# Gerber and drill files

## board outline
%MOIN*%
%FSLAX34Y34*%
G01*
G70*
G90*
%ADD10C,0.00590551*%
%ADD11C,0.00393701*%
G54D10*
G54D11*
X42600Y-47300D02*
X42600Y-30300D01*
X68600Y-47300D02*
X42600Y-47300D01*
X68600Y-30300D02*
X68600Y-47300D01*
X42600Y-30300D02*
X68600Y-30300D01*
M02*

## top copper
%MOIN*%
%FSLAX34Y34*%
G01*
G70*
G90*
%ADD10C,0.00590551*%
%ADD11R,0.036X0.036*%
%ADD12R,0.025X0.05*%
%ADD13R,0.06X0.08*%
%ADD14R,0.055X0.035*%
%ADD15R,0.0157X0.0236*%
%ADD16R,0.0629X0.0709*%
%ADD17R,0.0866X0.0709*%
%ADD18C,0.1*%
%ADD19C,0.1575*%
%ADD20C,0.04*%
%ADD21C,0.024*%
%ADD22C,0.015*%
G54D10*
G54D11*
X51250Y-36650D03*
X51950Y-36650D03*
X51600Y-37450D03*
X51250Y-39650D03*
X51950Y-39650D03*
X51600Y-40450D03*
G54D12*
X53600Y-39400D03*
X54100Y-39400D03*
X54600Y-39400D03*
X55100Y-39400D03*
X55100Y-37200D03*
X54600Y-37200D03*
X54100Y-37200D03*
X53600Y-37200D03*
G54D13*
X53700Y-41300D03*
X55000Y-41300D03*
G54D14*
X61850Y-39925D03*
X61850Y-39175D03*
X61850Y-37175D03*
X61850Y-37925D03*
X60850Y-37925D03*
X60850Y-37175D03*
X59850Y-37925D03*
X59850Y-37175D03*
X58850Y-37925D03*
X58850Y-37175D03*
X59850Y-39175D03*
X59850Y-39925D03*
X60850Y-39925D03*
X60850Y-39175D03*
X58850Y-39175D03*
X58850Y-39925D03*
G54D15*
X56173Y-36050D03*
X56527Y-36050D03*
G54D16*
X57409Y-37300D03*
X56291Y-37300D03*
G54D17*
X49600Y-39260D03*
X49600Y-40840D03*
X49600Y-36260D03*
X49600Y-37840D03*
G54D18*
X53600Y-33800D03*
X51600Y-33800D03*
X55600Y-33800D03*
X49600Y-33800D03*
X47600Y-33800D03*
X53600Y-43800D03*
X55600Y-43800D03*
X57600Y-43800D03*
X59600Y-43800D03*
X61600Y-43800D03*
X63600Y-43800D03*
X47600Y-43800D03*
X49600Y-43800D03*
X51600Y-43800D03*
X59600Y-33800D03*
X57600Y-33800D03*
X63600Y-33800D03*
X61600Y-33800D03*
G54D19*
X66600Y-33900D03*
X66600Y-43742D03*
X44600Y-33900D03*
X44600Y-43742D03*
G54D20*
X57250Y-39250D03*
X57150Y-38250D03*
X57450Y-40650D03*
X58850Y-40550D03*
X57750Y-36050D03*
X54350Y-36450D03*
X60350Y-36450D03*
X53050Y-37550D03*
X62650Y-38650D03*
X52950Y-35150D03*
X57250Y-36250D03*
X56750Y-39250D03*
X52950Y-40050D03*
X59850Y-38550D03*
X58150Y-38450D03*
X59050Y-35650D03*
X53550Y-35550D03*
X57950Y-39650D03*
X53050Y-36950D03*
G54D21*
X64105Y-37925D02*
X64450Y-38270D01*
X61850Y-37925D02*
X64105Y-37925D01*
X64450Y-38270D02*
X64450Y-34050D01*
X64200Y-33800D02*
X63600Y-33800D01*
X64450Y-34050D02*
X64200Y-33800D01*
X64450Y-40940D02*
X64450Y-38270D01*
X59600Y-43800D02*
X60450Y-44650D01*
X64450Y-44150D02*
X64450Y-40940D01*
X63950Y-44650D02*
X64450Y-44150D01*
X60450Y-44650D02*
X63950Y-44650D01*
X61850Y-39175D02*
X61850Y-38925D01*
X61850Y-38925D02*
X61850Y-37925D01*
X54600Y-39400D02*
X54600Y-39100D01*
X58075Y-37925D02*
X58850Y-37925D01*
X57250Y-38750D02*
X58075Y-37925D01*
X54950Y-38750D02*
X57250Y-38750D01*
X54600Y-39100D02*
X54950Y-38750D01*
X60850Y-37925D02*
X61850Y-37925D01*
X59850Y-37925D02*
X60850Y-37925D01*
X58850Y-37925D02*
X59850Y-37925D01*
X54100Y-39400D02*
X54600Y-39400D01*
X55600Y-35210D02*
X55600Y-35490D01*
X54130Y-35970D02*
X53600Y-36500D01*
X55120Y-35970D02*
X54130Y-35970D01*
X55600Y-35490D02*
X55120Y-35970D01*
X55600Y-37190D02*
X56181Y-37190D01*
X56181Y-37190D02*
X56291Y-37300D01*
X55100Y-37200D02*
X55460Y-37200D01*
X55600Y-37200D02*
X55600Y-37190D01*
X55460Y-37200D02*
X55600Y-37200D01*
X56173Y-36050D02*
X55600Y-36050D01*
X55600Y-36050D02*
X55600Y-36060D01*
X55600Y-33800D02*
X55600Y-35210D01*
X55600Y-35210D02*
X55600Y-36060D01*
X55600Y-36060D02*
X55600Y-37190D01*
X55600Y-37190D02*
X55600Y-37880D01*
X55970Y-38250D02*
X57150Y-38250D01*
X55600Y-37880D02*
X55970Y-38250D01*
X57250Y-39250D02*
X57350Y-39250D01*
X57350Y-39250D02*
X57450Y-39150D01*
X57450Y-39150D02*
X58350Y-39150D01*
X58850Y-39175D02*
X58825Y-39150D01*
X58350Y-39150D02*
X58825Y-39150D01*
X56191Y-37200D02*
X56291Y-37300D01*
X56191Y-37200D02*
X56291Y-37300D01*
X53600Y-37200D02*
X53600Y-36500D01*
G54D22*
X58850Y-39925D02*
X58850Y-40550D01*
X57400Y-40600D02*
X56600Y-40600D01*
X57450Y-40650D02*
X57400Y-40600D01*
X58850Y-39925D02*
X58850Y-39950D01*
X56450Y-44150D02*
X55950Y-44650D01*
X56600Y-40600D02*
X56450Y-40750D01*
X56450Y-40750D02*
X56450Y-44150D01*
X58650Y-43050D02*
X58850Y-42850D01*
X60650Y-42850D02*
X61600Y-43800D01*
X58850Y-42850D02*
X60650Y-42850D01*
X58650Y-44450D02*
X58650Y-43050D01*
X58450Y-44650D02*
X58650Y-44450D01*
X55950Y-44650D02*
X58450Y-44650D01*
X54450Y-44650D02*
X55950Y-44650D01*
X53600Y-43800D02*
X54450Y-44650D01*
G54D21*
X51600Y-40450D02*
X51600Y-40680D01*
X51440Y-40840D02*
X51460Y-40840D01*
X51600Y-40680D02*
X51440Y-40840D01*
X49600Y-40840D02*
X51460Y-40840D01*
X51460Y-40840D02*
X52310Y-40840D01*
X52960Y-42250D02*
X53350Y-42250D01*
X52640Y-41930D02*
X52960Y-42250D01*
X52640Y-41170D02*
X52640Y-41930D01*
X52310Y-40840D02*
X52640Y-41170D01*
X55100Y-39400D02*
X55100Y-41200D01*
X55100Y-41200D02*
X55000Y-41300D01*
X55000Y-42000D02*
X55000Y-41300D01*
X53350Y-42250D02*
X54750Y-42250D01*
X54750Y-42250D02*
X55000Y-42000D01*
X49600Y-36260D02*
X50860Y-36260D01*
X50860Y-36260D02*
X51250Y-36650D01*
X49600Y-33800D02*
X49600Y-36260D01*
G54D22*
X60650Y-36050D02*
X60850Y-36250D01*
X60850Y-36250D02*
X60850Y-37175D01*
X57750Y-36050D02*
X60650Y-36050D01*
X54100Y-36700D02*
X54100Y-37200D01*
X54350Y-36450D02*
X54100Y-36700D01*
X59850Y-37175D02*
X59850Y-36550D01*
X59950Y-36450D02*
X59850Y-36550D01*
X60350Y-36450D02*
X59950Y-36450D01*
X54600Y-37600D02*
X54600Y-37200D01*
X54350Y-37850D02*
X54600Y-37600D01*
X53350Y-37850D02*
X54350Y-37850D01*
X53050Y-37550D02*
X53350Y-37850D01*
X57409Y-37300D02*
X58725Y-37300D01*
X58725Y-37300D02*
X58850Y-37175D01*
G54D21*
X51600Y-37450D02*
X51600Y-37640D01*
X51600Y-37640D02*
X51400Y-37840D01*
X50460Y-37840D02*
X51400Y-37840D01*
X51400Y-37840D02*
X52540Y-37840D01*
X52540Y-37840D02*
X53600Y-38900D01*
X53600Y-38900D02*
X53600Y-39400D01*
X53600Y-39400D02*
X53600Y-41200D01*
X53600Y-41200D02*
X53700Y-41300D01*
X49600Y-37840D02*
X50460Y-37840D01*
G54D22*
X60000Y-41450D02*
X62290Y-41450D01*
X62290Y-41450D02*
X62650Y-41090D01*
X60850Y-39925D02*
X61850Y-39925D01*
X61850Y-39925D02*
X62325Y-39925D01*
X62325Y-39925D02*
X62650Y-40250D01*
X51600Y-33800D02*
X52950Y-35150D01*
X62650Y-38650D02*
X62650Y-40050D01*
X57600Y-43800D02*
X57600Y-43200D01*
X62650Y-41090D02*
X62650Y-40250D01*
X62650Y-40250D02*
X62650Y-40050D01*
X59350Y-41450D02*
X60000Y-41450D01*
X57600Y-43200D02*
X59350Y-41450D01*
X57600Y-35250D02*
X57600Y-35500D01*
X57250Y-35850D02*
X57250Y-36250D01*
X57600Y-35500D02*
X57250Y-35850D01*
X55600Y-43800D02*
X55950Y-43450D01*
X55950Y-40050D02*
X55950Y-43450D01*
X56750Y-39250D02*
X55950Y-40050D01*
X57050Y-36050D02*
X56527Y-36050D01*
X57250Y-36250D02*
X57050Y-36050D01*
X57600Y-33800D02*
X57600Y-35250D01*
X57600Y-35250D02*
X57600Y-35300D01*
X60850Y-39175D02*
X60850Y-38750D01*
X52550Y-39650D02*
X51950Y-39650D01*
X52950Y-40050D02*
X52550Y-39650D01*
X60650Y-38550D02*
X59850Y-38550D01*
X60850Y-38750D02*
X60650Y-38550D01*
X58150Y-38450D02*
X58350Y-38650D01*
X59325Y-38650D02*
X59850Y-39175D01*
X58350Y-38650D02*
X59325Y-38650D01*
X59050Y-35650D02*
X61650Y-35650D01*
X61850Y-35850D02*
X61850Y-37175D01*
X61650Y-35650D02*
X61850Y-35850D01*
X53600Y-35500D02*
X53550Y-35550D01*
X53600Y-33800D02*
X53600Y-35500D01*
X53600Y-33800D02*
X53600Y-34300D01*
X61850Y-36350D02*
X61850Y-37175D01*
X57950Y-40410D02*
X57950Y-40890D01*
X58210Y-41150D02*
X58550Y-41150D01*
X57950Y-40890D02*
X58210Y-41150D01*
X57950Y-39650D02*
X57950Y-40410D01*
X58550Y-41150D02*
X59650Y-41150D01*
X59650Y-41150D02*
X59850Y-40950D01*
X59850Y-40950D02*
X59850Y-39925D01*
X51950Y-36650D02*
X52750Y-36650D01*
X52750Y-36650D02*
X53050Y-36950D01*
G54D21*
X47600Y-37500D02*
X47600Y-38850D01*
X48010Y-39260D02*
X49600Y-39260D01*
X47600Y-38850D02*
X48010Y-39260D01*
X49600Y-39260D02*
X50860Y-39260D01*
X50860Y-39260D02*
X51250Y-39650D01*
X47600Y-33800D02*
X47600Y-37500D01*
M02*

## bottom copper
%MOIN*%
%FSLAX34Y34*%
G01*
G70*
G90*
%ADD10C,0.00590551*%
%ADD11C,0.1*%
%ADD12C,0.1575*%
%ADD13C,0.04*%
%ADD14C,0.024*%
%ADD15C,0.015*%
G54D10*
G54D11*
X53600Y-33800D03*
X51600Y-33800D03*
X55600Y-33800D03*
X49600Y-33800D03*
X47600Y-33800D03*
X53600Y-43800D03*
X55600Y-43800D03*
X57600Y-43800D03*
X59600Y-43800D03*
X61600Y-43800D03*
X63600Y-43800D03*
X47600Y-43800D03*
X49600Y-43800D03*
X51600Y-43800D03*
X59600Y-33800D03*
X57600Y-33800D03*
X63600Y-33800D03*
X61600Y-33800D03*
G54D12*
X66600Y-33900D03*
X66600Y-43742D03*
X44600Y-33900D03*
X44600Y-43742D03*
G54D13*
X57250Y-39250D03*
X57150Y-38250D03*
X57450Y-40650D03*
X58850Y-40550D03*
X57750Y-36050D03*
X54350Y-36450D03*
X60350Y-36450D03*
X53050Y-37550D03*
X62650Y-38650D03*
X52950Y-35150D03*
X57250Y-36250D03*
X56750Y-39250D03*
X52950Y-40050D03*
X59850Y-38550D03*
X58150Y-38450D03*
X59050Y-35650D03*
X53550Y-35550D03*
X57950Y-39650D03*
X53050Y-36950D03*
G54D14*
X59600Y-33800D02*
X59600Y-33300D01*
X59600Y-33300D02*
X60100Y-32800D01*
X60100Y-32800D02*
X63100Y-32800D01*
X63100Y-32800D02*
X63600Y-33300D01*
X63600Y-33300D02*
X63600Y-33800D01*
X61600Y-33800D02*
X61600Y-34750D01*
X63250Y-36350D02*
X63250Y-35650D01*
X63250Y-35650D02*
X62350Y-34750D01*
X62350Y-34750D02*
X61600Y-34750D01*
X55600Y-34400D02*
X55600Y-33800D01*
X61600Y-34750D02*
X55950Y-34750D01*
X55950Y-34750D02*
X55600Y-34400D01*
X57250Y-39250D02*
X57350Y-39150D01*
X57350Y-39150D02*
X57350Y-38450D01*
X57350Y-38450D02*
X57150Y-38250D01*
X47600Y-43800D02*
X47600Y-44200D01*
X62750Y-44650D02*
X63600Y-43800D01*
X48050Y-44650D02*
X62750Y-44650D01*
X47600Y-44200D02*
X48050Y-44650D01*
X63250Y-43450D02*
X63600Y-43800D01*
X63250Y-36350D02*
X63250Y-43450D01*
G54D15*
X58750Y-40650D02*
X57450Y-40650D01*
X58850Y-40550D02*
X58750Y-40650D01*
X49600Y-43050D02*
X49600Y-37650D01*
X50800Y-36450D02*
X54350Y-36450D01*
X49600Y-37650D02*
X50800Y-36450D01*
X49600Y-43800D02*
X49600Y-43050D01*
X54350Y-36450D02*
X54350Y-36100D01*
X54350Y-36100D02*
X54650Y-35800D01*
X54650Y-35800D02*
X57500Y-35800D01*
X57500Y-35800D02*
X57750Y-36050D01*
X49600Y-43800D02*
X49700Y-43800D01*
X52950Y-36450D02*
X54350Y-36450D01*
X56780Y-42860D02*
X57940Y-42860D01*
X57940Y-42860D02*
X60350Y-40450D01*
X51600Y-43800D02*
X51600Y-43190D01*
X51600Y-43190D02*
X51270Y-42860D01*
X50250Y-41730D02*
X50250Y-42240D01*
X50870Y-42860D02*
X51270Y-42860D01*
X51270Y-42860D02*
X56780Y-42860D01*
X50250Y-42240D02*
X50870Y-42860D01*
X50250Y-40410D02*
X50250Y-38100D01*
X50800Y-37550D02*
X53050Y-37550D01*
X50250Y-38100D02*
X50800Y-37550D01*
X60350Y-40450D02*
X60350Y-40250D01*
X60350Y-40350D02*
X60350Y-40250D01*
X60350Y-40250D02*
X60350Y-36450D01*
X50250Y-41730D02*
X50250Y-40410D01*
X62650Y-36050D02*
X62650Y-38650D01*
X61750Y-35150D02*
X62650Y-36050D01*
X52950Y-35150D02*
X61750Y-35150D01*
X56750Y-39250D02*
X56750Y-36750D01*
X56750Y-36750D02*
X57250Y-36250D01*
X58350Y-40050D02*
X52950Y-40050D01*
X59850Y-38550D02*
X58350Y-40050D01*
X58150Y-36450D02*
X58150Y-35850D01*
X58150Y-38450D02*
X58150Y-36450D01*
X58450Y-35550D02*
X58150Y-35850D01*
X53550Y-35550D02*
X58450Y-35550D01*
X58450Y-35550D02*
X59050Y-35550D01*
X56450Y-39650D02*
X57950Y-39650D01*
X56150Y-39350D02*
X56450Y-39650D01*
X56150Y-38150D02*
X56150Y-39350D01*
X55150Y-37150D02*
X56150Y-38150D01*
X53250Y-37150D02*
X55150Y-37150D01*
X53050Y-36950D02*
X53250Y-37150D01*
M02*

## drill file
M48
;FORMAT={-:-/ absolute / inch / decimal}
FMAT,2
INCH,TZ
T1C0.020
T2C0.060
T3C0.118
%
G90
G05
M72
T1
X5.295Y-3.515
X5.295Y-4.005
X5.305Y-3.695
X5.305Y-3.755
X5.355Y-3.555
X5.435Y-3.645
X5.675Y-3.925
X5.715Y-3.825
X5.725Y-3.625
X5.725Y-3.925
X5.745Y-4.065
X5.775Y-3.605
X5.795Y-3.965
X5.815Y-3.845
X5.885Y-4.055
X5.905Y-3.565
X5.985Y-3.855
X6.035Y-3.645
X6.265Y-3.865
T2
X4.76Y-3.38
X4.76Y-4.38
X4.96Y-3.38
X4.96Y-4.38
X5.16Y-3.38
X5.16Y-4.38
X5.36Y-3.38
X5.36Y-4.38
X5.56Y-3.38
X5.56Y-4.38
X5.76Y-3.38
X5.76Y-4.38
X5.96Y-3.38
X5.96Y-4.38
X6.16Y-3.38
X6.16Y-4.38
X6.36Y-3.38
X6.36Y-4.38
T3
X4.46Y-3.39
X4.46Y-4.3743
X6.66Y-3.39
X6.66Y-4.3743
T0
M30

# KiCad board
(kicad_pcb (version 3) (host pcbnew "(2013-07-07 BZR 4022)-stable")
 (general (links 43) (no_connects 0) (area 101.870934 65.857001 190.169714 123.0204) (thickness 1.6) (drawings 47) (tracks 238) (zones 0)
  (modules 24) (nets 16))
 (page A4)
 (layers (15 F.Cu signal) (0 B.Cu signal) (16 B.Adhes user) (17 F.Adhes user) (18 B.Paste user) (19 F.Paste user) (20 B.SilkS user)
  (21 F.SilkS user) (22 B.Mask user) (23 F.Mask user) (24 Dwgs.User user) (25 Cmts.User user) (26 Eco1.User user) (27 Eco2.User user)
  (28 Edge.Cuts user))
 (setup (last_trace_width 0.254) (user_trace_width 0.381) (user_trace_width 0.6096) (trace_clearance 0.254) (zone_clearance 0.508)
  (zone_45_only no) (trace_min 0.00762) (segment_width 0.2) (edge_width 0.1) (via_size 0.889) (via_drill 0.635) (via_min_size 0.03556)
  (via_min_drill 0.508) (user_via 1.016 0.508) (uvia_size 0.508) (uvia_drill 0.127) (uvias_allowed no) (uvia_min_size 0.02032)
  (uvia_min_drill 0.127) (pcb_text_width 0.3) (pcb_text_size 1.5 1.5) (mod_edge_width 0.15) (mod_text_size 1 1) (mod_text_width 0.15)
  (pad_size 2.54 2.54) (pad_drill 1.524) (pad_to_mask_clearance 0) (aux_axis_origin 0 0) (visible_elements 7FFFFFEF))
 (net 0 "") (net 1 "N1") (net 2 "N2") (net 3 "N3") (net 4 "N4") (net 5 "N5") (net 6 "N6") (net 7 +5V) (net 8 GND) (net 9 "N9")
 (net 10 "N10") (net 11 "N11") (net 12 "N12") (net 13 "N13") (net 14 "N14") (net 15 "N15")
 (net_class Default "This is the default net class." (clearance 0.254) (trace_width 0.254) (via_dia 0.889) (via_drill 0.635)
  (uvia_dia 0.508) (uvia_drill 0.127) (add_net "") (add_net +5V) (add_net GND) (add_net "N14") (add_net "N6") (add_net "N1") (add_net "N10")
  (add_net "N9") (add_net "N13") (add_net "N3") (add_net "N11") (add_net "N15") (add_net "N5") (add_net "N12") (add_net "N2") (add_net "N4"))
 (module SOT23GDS (layer F.Cu) (at 131.064 94.107)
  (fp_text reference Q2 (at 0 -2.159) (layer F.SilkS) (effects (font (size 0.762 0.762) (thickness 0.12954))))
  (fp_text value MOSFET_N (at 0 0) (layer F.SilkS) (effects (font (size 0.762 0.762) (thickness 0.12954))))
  (pad S smd rect (at -0.889 -1.016) (size 0.9144 0.9144) (layers F.Cu F.Paste F.Mask) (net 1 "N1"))
  (pad G smd rect (at 0.889 -1.016) (size 0.9144 0.9144) (layers F.Cu F.Paste F.Mask) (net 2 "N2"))
  (pad D smd rect (at 0 1.016) (size 0.9144 0.9144) (layers F.Cu F.Paste F.Mask) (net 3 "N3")))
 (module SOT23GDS (layer F.Cu) (at 131.064 101.727)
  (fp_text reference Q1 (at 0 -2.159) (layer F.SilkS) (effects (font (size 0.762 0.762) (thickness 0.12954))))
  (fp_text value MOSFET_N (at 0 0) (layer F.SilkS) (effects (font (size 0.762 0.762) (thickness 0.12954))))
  (pad S smd rect (at -0.889 -1.016) (size 0.9144 0.9144) (layers F.Cu F.Paste F.Mask) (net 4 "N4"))
  (pad G smd rect (at 0.889 -1.016) (size 0.9144 0.9144) (layers F.Cu F.Paste F.Mask) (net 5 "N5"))
  (pad D smd rect (at 0 1.016) (size 0.9144 0.9144) (layers F.Cu F.Paste F.Mask) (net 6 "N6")))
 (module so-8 (layer F.Cu) (at 138.049 97.282)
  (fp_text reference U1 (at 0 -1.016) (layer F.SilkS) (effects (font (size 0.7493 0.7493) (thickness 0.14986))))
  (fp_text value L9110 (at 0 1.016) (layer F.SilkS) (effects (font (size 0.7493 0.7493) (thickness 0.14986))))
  (pad 1 smd rect (at -1.905 2.794) (size 0.635 1.27) (layers F.Cu F.Paste F.Mask) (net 3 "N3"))
  (pad 2 smd rect (at -0.635 2.794) (size 0.635 1.27) (layers F.Cu F.Paste F.Mask) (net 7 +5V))
  (pad 3 smd rect (at 0.635 2.794) (size 0.635 1.27) (layers F.Cu F.Paste F.Mask) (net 7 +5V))
  (pad 4 smd rect (at 1.905 2.794) (size 0.635 1.27) (layers F.Cu F.Paste F.Mask) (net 6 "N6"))
  (pad 5 smd rect (at 1.905 -2.794) (size 0.635 1.27) (layers F.Cu F.Paste F.Mask) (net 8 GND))
  (pad 6 smd rect (at 0.635 -2.794) (size 0.635 1.27) (layers F.Cu F.Paste F.Mask) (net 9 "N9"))
  (pad 7 smd rect (at -0.635 -2.794) (size 0.635 1.27) (layers F.Cu F.Paste F.Mask) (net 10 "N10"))
  (pad 8 smd rect (at -1.905 -2.794) (size 0.635 1.27) (layers F.Cu F.Paste F.Mask) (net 8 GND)))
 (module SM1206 (layer F.Cu) (at 138.049 104.902)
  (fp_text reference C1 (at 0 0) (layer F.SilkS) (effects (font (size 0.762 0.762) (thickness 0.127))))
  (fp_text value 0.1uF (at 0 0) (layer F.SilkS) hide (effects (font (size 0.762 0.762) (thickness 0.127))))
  (pad 1 smd rect (at -1.651 0) (size 1.524 2.032) (layers F.Cu F.Paste F.Mask) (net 3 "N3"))
  (pad 2 smd rect (at 1.651 0) (size 1.524 2.032) (layers F.Cu F.Paste F.Mask) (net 6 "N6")))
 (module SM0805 (layer F.Cu) (at 157.099 100.457 90)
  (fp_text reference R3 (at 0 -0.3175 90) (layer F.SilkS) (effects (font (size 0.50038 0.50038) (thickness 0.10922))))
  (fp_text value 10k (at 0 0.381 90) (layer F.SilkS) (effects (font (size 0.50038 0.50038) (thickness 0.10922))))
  (pad 1 smd rect (at -0.9525 0 90) (size 0.889 1.397) (layers F.Cu F.Paste F.Mask) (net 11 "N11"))
  (pad 2 smd rect (at 0.9525 0 90) (size 0.889 1.397) (layers F.Cu F.Paste F.Mask) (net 7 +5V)))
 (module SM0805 (layer F.Cu) (at 157.099 95.377 270)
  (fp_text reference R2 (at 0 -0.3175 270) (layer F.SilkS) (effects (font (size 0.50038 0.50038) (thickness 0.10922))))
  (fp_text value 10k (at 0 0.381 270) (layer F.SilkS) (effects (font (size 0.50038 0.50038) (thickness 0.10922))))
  (pad 1 smd rect (at -0.9525 0 270) (size 0.889 1.397) (layers F.Cu F.Paste F.Mask) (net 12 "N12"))
  (pad 2 smd rect (at 0.9525 0 270) (size 0.889 1.397) (layers F.Cu F.Paste F.Mask) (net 7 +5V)))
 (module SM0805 (layer F.Cu) (at 154.559 95.377 90)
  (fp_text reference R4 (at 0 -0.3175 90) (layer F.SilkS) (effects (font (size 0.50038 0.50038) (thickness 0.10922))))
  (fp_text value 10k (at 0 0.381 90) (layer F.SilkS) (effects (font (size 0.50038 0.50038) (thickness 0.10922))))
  (pad 1 smd rect (at -0.9525 0 90) (size 0.889 1.397) (layers F.Cu F.Paste F.Mask) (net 7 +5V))
  (pad 2 smd rect (at 0.9525 0 90) (size 0.889 1.397) (layers F.Cu F.Paste F.Mask) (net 10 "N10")))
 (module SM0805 (layer F.Cu) (at 152.019 95.377 90)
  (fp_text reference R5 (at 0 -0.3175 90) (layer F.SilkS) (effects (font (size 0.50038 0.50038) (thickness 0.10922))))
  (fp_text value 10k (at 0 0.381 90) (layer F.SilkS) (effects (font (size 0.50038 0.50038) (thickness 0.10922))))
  (pad 1 smd rect (at -0.9525 0 90) (size 0.889 1.397) (layers F.Cu F.Paste F.Mask) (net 7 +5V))
  (pad 2 smd rect (at 0.9525 0 90) (size 0.889 1.397) (layers F.Cu F.Paste F.Mask) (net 9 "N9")))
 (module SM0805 (layer F.Cu) (at 149.479 95.377 90)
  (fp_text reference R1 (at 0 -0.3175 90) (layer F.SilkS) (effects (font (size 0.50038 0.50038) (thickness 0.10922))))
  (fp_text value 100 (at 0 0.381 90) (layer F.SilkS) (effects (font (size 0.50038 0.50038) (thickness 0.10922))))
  (pad 1 smd rect (at -0.9525 0 90) (size 0.889 1.397) (layers F.Cu F.Paste F.Mask) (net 7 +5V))
  (pad 2 smd rect (at 0.9525 0 90) (size 0.889 1.397) (layers F.Cu F.Paste F.Mask) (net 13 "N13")))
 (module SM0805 (layer F.Cu) (at 152.019 100.457 270)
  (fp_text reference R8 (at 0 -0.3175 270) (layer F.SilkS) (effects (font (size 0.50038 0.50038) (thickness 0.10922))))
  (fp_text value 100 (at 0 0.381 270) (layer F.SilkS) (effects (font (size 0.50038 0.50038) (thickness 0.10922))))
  (pad 1 smd rect (at -0.9525 0 270) (size 0.889 1.397) (layers F.Cu F.Paste F.Mask) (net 12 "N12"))
  (pad 2 smd rect (at 0.9525 0 270) (size 0.889 1.397) (layers F.Cu F.Paste F.Mask) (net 2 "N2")))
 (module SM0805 (layer F.Cu) (at 154.559 100.457 90)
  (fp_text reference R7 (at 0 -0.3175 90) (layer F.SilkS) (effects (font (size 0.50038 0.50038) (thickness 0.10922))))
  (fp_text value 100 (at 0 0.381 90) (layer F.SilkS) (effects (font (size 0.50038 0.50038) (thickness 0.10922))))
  (pad 1 smd rect (at -0.9525 0 90) (size 0.889 1.397) (layers F.Cu F.Paste F.Mask) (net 11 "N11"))
  (pad 2 smd rect (at 0.9525 0 90) (size 0.889 1.397) (layers F.Cu F.Paste F.Mask) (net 5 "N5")))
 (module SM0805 (layer F.Cu) (at 149.479 100.457 270)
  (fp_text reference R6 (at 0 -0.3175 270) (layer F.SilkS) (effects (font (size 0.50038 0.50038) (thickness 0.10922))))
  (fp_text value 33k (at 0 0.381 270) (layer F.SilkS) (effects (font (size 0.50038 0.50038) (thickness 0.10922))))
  (pad 1 smd rect (at -0.9525 0 270) (size 0.889 1.397) (layers F.Cu F.Paste F.Mask) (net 8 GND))
  (pad 2 smd rect (at 0.9525 0 270) (size 0.889 1.397) (layers F.Cu F.Paste F.Mask) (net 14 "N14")))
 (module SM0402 (layer F.Cu) (at 143.129 91.567)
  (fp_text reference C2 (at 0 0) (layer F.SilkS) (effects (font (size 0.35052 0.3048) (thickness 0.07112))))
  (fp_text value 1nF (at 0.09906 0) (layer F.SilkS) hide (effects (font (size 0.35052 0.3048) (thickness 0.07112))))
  (pad 1 smd rect (at -0.44958 0) (size 0.39878 0.59944) (layers F.Cu F.Paste F.Mask) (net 8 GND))
  (pad 2 smd rect (at 0.44958 0) (size 0.39878 0.59944) (layers F.Cu F.Paste F.Mask) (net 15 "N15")))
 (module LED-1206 (layer F.Cu) (at 144.399 94.742 180)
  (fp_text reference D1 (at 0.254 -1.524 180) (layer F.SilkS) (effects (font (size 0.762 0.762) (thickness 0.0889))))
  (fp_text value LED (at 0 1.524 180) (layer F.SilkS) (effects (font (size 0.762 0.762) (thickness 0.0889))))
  (pad 1 smd rect (at -1.41986 0 180) (size 1.59766 1.80086) (layers F.Cu F.Paste F.Mask) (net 13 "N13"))
  (pad 2 smd rect (at 1.41986 0 180) (size 1.59766 1.80086) (layers F.Cu F.Paste F.Mask) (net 8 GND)))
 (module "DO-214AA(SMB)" (layer F.Cu) (at 125.984 101.727 270)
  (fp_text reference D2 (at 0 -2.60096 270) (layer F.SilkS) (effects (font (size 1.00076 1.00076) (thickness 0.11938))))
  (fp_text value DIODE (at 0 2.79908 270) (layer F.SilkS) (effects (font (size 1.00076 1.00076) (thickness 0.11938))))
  (pad 1 smd rect (at -2.0066 0 270) (size 1.80086 2.19964) (layers F.Cu F.Paste F.Mask) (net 4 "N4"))
  (pad 2 smd rect (at 2.0066 0 270) (size 1.80086 2.19964) (layers F.Cu F.Paste F.Mask) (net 6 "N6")))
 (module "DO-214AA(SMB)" (layer F.Cu) (at 125.984 94.107 270)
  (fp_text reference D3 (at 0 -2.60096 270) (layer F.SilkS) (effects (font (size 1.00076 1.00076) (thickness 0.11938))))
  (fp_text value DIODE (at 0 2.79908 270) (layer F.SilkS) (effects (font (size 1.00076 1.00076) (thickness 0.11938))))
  (pad 1 smd rect (at -2.0066 0 270) (size 1.80086 2.19964) (layers F.Cu F.Paste F.Mask) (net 1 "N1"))
  (pad 2 smd rect (at 2.0066 0 270) (size 1.80086 2.19964) (layers F.Cu F.Paste F.Mask) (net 3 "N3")))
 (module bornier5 (layer F.Cu) (at 131.064 85.852 180)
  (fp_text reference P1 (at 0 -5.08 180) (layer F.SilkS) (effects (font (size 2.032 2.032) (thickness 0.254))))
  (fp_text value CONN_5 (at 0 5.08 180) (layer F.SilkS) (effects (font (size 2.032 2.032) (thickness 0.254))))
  (pad 2 thru_hole circle (at -5.08 0 180) (size 2.54 2.54) (drill 1.524) (layers *.Cu *.Mask F.SilkS) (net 12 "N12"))
  (pad 3 thru_hole circle (at 0 0 180) (size 2.54 2.54) (drill 1.524) (layers *.Cu *.Mask F.SilkS) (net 11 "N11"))
  (pad 1 thru_hole circle (at -10.16 0 180) (size 2.54 2.54) (drill 1.524) (layers *.Cu *.Mask F.SilkS) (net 8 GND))
  (pad 4 thru_hole circle (at 5.08 0 180) (size 2.54 2.54) (drill 1.524) (layers *.Cu *.Mask F.SilkS) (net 1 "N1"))
  (pad 5 thru_hole circle (at 10.16 0 180) (size 2.54 2.54) (drill 1.524) (layers *.Cu *.Mask F.SilkS) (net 4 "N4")))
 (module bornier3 (layer F.Cu) (at 141.224 111.252)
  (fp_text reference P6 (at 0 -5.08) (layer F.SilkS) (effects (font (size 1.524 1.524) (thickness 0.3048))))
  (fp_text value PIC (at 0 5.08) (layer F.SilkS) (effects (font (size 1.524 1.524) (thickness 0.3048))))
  (pad 1 thru_hole circle (at -5.08 0) (size 2.54 2.54) (drill 1.524) (layers *.Cu *.Mask F.SilkS) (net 14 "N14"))
  (pad 2 thru_hole circle (at 0 0) (size 2.54 2.54) (drill 1.524) (layers *.Cu *.Mask F.SilkS) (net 15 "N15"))
  (pad 3 thru_hole circle (at 5.08 0) (size 2.54 2.54) (drill 1.524) (layers *.Cu *.Mask F.SilkS) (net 11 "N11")))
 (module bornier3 (layer F.Cu) (at 156.464 111.252)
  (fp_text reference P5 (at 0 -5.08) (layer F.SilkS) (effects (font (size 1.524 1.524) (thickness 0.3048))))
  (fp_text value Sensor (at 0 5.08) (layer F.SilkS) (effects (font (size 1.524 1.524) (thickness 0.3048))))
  (pad 1 thru_hole circle (at -5.08 0) (size 2.54 2.54) (drill 1.524) (layers *.Cu *.Mask F.SilkS) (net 7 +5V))
  (pad 2 thru_hole circle (at 0 0) (size 2.54 2.54) (drill 1.524) (layers *.Cu *.Mask F.SilkS) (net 14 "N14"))
  (pad 3 thru_hole circle (at 5.08 0) (size 2.54 2.54) (drill 1.524) (layers *.Cu *.Mask F.SilkS) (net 8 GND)))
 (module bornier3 (layer F.Cu) (at 125.984 111.252)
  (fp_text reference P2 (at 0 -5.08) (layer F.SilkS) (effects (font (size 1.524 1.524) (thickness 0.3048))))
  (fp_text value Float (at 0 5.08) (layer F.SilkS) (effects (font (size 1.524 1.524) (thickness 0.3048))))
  (pad 1 thru_hole circle (at -5.08 0) (size 2.54 2.54) (drill 1.524) (layers *.Cu *.Mask F.SilkS) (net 8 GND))
  (pad 2 thru_hole circle (at 0 0) (size 2.54 2.54) (drill 1.524) (layers *.Cu *.Mask F.SilkS) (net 10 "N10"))
  (pad 3 thru_hole circle (at 5.08 0) (size 2.54 2.54) (drill 1.524) (layers *.Cu *.Mask F.SilkS) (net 9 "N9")))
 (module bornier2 (layer F.Cu) (at 148.844 85.852 180)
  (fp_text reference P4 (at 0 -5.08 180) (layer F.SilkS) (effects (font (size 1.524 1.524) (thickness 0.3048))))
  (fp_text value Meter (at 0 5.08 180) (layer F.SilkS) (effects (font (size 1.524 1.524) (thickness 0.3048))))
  (pad 1 thru_hole circle (at -2.54 0 180) (size 2.54 2.54) (drill 1.524) (layers *.Cu *.Mask F.SilkS) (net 7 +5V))
  (pad 2 thru_hole circle (at 2.54 0 180) (size 2.54 2.54) (drill 1.524) (layers *.Cu *.Mask F.SilkS) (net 15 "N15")))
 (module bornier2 (layer F.Cu) (at 159.004 85.852 180)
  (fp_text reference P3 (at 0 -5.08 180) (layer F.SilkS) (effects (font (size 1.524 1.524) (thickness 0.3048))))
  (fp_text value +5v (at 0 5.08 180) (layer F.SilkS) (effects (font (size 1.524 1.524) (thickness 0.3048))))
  (pad 1 thru_hole circle (at -2.54 0 180) (size 2.54 2.54) (drill 1.524) (layers *.Cu *.Mask F.SilkS) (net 7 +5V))
  (pad 2 thru_hole circle (at 2.54 0 180) (size 2.54 2.54) (drill 1.524) (layers *.Cu *.Mask F.SilkS) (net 8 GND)))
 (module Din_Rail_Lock (layer F.Cu) (at 169.164 86.106)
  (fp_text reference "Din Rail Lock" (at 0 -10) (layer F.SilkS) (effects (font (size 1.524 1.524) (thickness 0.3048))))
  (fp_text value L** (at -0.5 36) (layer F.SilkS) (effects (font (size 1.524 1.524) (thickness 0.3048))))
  (pad 1 thru_hole circle (at 0 0) (size 4.0005 4.0005) (drill 3) (layers *.Cu *.Mask F.SilkS))
  (pad 2 thru_hole circle (at 0 25) (size 4.0005 4.0005) (drill 3) (layers *.Cu *.Mask F.SilkS)))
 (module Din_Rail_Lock (layer F.Cu) (at 113.284 86.106)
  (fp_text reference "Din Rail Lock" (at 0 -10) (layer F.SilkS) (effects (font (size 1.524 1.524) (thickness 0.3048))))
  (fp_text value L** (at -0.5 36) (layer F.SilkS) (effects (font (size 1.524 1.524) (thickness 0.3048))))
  (pad 1 thru_hole circle (at 0 0) (size 4.0005 4.0005) (drill 3) (layers *.Cu *.Mask F.SilkS))
  (pad 2 thru_hole circle (at 0 25) (size 4.0005 4.0005) (drill 3) (layers *.Cu *.Mask F.SilkS)))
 (gr_line (start 108.204 120.142) (end 108.204 76.962) (angle 90) (layer Edge.Cuts) (width 0.1))
 (gr_line (start 174.244 120.142) (end 108.204 120.142) (angle 90) (layer Edge.Cuts) (width 0.1))
 (gr_line (start 174.244 76.962) (end 174.244 120.142) (angle 90) (layer Edge.Cuts) (width 0.1))
 (gr_line (start 108.204 76.962) (end 174.244 76.962) (angle 90) (layer Edge.Cuts) (width 0.1))
 (segment (start 162.8267 96.3295) (end 163.703 97.2058) (width 0.6096) (layer F.Cu) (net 7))
 (segment (start 157.099 96.3295) (end 162.8267 96.3295) (width 0.6096) (layer F.Cu) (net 7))
 (segment (start 163.703 97.2058) (end 163.703 86.487) (width 0.6096) (layer F.Cu) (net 7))
 (segment (start 163.068 85.852) (end 161.544 85.852) (width 0.6096) (layer F.Cu) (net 7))
 (segment (start 163.703 86.487) (end 163.068 85.852) (width 0.6096) (layer F.Cu) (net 7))
 (segment (start 163.703 103.9876) (end 163.703 97.2058) (width 0.6096) (layer F.Cu) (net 7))
 (segment (start 151.384 111.252) (end 153.543 113.411) (width 0.6096) (layer F.Cu) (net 7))
 (segment (start 163.703 112.141) (end 163.703 103.9876) (width 0.6096) (layer F.Cu) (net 7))
 (segment (start 162.433 113.411) (end 163.703 112.141) (width 0.6096) (layer F.Cu) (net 7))
 (segment (start 153.543 113.411) (end 162.433 113.411) (width 0.6096) (layer F.Cu) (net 7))
 (segment (start 157.099 99.5045) (end 157.099 98.8695) (width 0.6096) (layer F.Cu) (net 7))
 (segment (start 157.099 98.8695) (end 157.099 96.3295) (width 0.6096) (layer F.Cu) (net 7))
 (segment (start 138.684 100.076) (end 138.684 99.314) (width 0.6096) (layer F.Cu) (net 7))
 (segment (start 147.5105 96.3295) (end 149.479 96.3295) (width 0.6096) (layer F.Cu) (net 7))
 (segment (start 145.415 98.425) (end 147.5105 96.3295) (width 0.6096) (layer F.Cu) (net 7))
 (segment (start 139.573 98.425) (end 145.415 98.425) (width 0.6096) (layer F.Cu) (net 7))
 (segment (start 138.684 99.314) (end 139.573 98.425) (width 0.6096) (layer F.Cu) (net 7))
 (segment (start 154.559 96.3295) (end 157.099 96.3295) (width 0.6096) (layer F.Cu) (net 7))
 (segment (start 152.019 96.3295) (end 154.559 96.3295) (width 0.6096) (layer F.Cu) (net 7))
 (segment (start 149.479 96.3295) (end 152.019 96.3295) (width 0.6096) (layer F.Cu) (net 7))
 (segment (start 137.414 100.076) (end 138.684 100.076) (width 0.6096) (layer F.Cu) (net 7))
 (segment (start 151.384 85.852) (end 151.384 84.582) (width 0.6096) (layer B.Cu) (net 7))
 (segment (start 151.384 84.582) (end 152.654 83.312) (width 0.6096) (layer B.Cu) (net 7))
 (segment (start 152.654 83.312) (end 160.274 83.312) (width 0.6096) (layer B.Cu) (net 7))
 (segment (start 160.274 83.312) (end 161.544 84.582) (width 0.6096) (layer B.Cu) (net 7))
 (segment (start 161.544 84.582) (end 161.544 85.852) (width 0.6096) (layer B.Cu) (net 7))
 (segment (start 156.464 85.852) (end 156.464 88.265) (width 0.6096) (layer B.Cu) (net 8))
 (segment (start 160.655 92.329) (end 160.655 90.551) (width 0.6096) (layer B.Cu) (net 8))
 (segment (start 160.655 90.551) (end 158.369 88.265) (width 0.6096) (layer B.Cu) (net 8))
 (segment (start 158.369 88.265) (end 156.464 88.265) (width 0.6096) (layer B.Cu) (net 8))
 (segment (start 141.224 87.376) (end 141.224 85.852) (width 0.6096) (layer B.Cu) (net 8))
 (segment (start 156.464 88.265) (end 142.113 88.265) (width 0.6096) (layer B.Cu) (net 8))
 (segment (start 142.113 88.265) (end 141.224 87.376) (width 0.6096) (layer B.Cu) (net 8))
 (segment (start 141.224 89.4334) (end 141.224 90.1446) (width 0.6096) (layer F.Cu) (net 8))
 (segment (start 137.4902 91.3638) (end 136.144 92.71) (width 0.6096) (layer F.Cu) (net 8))
 (segment (start 140.0048 91.3638) (end 137.4902 91.3638) (width 0.6096) (layer F.Cu) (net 8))
 (segment (start 141.224 90.1446) (end 140.0048 91.3638) (width 0.6096) (layer F.Cu) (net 8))
 (segment (start 141.224 94.4626) (end 142.69974 94.4626) (width 0.6096) (layer F.Cu) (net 8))
 (segment (start 142.69974 94.4626) (end 142.97914 94.742) (width 0.6096) (layer F.Cu) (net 8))
 (segment (start 139.954 94.488) (end 140.8684 94.488) (width 0.6096) (layer F.Cu) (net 8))
 (segment (start 141.224 94.488) (end 141.224 94.4626) (width 0.6096) (layer F.Cu) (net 8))
 (segment (start 140.8684 94.488) (end 141.224 94.488) (width 0.6096) (layer F.Cu) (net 8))
 (segment (start 142.67942 91.567) (end 141.224 91.567) (width 0.6096) (layer F.Cu) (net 8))
 (segment (start 141.224 91.567) (end 141.224 91.5924) (width 0.6096) (layer F.Cu) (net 8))
 (segment (start 141.224 85.852) (end 141.224 89.4334) (width 0.6096) (layer F.Cu) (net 8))
 (segment (start 141.224 89.4334) (end 141.224 91.5924) (width 0.6096) (layer F.Cu) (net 8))
 (segment (start 141.224 91.5924) (end 141.224 94.4626) (width 0.6096) (layer F.Cu) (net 8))
 (segment (start 141.224 94.4626) (end 141.224 96.2152) (width 0.6096) (layer F.Cu) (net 8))
 (segment (start 142.1638 97.155) (end 145.161 97.155) (width 0.6096) (layer F.Cu) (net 8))
 (segment (start 141.224 96.2152) (end 142.1638 97.155) (width 0.6096) (layer F.Cu) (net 8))
 (segment (start 145.415 99.695) (end 145.669 99.695) (width 0.6096) (layer F.Cu) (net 8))
 (segment (start 145.669 99.695) (end 145.923 99.441) (width 0.6096) (layer F.Cu) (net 8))
 (segment (start 145.923 99.441) (end 148.209 99.441) (width 0.6096) (layer F.Cu) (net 8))
 (via blind (at 145.415 99.695) (size 1.016) (drill 0.508) (layers F.Cu B.Cu) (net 8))
 (segment (start 145.415 99.695) (end 145.669 99.441) (width 0.6096) (layer B.Cu) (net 8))
 (segment (start 145.669 99.441) (end 145.669 97.663) (width 0.6096) (layer B.Cu) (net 8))
 (segment (start 145.669 97.663) (end 145.161 97.155) (width 0.6096) (layer B.Cu) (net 8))
 (via blind (at 145.161 97.155) (size 1.016) (drill 0.508) (layers F.Cu B.Cu) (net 8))
 (segment (start 149.479 99.5045) (end 149.4155 99.441) (width 0.6096) (layer F.Cu) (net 8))
 (segment (start 148.209 99.441) (end 149.4155 99.441) (width 0.6096) (layer F.Cu) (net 8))
 (segment (start 142.72514 94.488) (end 142.97914 94.742) (width 0.6096) (layer F.Cu) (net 8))
 (segment (start 142.72514 94.488) (end 142.97914 94.742) (width 0.6096) (layer F.Cu) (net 8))
 (segment (start 136.144 94.488) (end 136.144 92.71) (width 0.6096) (layer F.Cu) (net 8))
 (segment (start 120.904 111.252) (end 120.904 112.268) (width 0.6096) (layer B.Cu) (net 8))
 (segment (start 159.385 113.411) (end 161.544 111.252) (width 0.6096) (layer B.Cu) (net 8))
 (segment (start 122.047 113.411) (end 159.385 113.411) (width 0.6096) (layer B.Cu) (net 8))
 (segment (start 120.904 112.268) (end 122.047 113.411) (width 0.6096) (layer B.Cu) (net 8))
 (segment (start 160.655 110.363) (end 161.544 111.252) (width 0.6096) (layer B.Cu) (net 8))
 (segment (start 160.655 92.329) (end 160.655 110.363) (width 0.6096) (layer B.Cu) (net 8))
 (segment (start 149.479 101.4095) (end 149.479 102.997) (width 0.381) (layer F.Cu) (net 14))
 (segment (start 145.796 103.124) (end 143.764 103.124) (width 0.381) (layer F.Cu) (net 14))
 (segment (start 145.923 103.251) (end 145.796 103.124) (width 0.381) (layer F.Cu) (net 14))
 (via blind (at 145.923 103.251) (size 1.016) (drill 0.508) (layers F.Cu B.Cu) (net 14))
 (segment (start 149.225 103.251) (end 145.923 103.251) (width 0.381) (layer B.Cu) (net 14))
 (segment (start 149.479 102.997) (end 149.225 103.251) (width 0.381) (layer B.Cu) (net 14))
 (via blind (at 149.479 102.997) (size 1.016) (drill 0.508) (layers F.Cu B.Cu) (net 14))
 (segment (start 149.479 101.4095) (end 149.479 101.473) (width 0.381) (layer F.Cu) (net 14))
 (segment (start 143.383 112.141) (end 142.113 113.411) (width 0.381) (layer F.Cu) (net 14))
 (segment (start 143.764 103.124) (end 143.383 103.505) (width 0.381) (layer F.Cu) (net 14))
 (segment (start 143.383 103.505) (end 143.383 112.141) (width 0.381) (layer F.Cu) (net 14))
 (segment (start 148.971 109.347) (end 149.479 108.839) (width 0.381) (layer F.Cu) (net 14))
 (segment (start 154.051 108.839) (end 156.464 111.252) (width 0.381) (layer F.Cu) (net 14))
 (segment (start 149.479 108.839) (end 154.051 108.839) (width 0.381) (layer F.Cu) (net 14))
 (segment (start 148.971 112.903) (end 148.971 109.347) (width 0.381) (layer F.Cu) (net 14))
 (segment (start 148.463 113.411) (end 148.971 112.903) (width 0.381) (layer F.Cu) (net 14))
 (segment (start 142.113 113.411) (end 148.463 113.411) (width 0.381) (layer F.Cu) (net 14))
 (segment (start 138.303 113.411) (end 142.113 113.411) (width 0.381) (layer F.Cu) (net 14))
 (segment (start 136.144 111.252) (end 138.303 113.411) (width 0.381) (layer F.Cu) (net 14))
 (segment (start 131.064 102.743) (end 131.064 103.3272) (width 0.6096) (layer F.Cu) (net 6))
 (segment (start 130.6576 103.7336) (end 130.7084 103.7336) (width 0.6096) (layer F.Cu) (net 6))
 (segment (start 131.064 103.3272) (end 130.6576 103.7336) (width 0.6096) (layer F.Cu) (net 6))
 (segment (start 125.984 103.7336) (end 130.7084 103.7336) (width 0.6096) (layer F.Cu) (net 6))
 (segment (start 130.7084 103.7336) (end 132.8674 103.7336) (width 0.6096) (layer F.Cu) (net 6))
 (segment (start 134.5184 107.315) (end 135.509 107.315) (width 0.6096) (layer F.Cu) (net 6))
 (segment (start 133.7056 106.5022) (end 134.5184 107.315) (width 0.6096) (layer F.Cu) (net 6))
 (segment (start 133.7056 104.5718) (end 133.7056 106.5022) (width 0.6096) (layer F.Cu) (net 6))
 (segment (start 132.8674 103.7336) (end 133.7056 104.5718) (width 0.6096) (layer F.Cu) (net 6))
 (segment (start 139.954 100.076) (end 139.954 104.648) (width 0.6096) (layer F.Cu) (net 6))
 (segment (start 139.954 104.648) (end 139.7 104.902) (width 0.6096) (layer F.Cu) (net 6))
 (segment (start 139.7 106.68) (end 139.7 104.902) (width 0.6096) (layer F.Cu) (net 6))
 (segment (start 135.509 107.315) (end 139.065 107.315) (width 0.6096) (layer F.Cu) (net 6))
 (segment (start 139.065 107.315) (end 139.7 106.68) (width 0.6096) (layer F.Cu) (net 6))
 (segment (start 125.984 92.1004) (end 129.1844 92.1004) (width 0.6096) (layer F.Cu) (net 1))
 (segment (start 129.1844 92.1004) (end 130.175 93.091) (width 0.6096) (layer F.Cu) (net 1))
 (segment (start 125.984 85.852) (end 125.984 92.1004) (width 0.6096) (layer F.Cu) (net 1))
 (segment (start 125.984 109.347) (end 125.984 95.631) (width 0.381) (layer B.Cu) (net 10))
 (segment (start 129.032 92.583) (end 138.049 92.583) (width 0.381) (layer B.Cu) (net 10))
 (segment (start 125.984 95.631) (end 129.032 92.583) (width 0.381) (layer B.Cu) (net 10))
 (segment (start 125.984 111.252) (end 125.984 109.347) (width 0.381) (layer B.Cu) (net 10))
 (segment (start 138.049 92.583) (end 138.049 91.694002) (width 0.381) (layer B.Cu) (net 10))
 (segment (start 138.049 91.694002) (end 138.811 90.932002) (width 0.381) (layer B.Cu) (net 10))
 (segment (start 138.811 90.932002) (end 146.050002 90.932002) (width 0.381) (layer B.Cu) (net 10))
 (segment (start 146.050002 90.932002) (end 146.685 91.567) (width 0.381) (layer B.Cu) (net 10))
 (segment (start 154.051 91.567) (end 154.559 92.075) (width 0.381) (layer F.Cu) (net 10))
 (segment (start 154.559 92.075) (end 154.559 94.4245) (width 0.381) (layer F.Cu) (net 10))
 (via blind (at 146.685 91.567) (size 1.016) (drill 0.508) (layers F.Cu B.Cu) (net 10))
 (segment (start 146.685 91.567) (end 154.051 91.567) (width 0.381) (layer F.Cu) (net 10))
 (segment (start 125.984 111.252) (end 126.238 111.252) (width 0.381) (layer B.Cu) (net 10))
 (segment (start 137.414 93.218) (end 137.414 94.488) (width 0.381) (layer F.Cu) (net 10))
 (via blind (at 138.049 92.583) (size 1.016) (drill 0.508) (layers F.Cu B.Cu) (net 10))
 (segment (start 138.049 92.583) (end 137.414 93.218) (width 0.381) (layer F.Cu) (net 10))
 (segment (start 134.493 92.583) (end 138.049 92.583) (width 0.381) (layer B.Cu) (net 10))
 (segment (start 144.2212 108.8644) (end 147.1676 108.8644) (width 0.381) (layer B.Cu) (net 9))
 (segment (start 147.1676 108.8644) (end 153.289 102.743) (width 0.381) (layer B.Cu) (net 9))
 (segment (start 131.064 111.252) (end 131.064 109.7026) (width 0.381) (layer B.Cu) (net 9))
 (segment (start 131.064 109.7026) (end 130.2258 108.8644) (width 0.381) (layer B.Cu) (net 9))
 (segment (start 127.635 105.9942) (end 127.635 107.2896) (width 0.381) (layer B.Cu) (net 9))
 (segment (start 129.2098 108.8644) (end 130.2258 108.8644) (width 0.381) (layer B.Cu) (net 9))
 (segment (start 130.2258 108.8644) (end 144.2212 108.8644) (width 0.381) (layer B.Cu) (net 9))
 (segment (start 127.635 107.2896) (end 129.2098 108.8644) (width 0.381) (layer B.Cu) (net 9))
 (segment (start 127.635 102.6414) (end 127.635 96.774) (width 0.381) (layer B.Cu) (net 9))
 (segment (start 129.032 95.377) (end 134.747 95.377) (width 0.381) (layer B.Cu) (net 9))
 (segment (start 127.635 96.774) (end 129.032 95.377) (width 0.381) (layer B.Cu) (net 9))
 (segment (start 153.289 102.743) (end 153.289 102.235) (width 0.381) (layer B.Cu) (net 9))
 (segment (start 153.289 102.489) (end 153.289 102.235) (width 0.381) (layer B.Cu) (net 9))
 (segment (start 153.289 102.235) (end 153.289 92.583) (width 0.381) (layer B.Cu) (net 9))
 (segment (start 152.019 94.4245) (end 152.019 92.837) (width 0.381) (layer F.Cu) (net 9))
 (segment (start 152.273 92.583) (end 152.019 92.837) (width 0.381) (layer F.Cu) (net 9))
 (segment (start 153.289 92.583) (end 152.273 92.583) (width 0.381) (layer F.Cu) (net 9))
 (via blind (at 153.289 92.583) (size 1.016) (drill 0.508) (layers F.Cu B.Cu) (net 9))
 (via blind (at 134.747 95.377) (size 1.016) (drill 0.508) (layers F.Cu B.Cu) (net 9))
 (segment (start 138.684 95.504) (end 138.684 94.488) (width 0.381) (layer F.Cu) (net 9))
 (segment (start 138.049 96.139) (end 138.684 95.504) (width 0.381) (layer F.Cu) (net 9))
 (segment (start 135.509 96.139) (end 138.049 96.139) (width 0.381) (layer F.Cu) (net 9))
 (segment (start 134.747 95.377) (end 135.509 96.139) (width 0.381) (layer F.Cu) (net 9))
 (segment (start 127.635 105.9942) (end 127.635 102.6414) (width 0.381) (layer B.Cu) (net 9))
 (segment (start 145.81886 94.742) (end 149.1615 94.742) (width 0.381) (layer F.Cu) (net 13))
 (segment (start 149.1615 94.742) (end 149.479 94.4245) (width 0.381) (layer F.Cu) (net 13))
 (segment (start 131.064 95.123) (end 131.064 95.6056) (width 0.6096) (layer F.Cu) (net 3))
 (segment (start 131.064 95.6056) (end 130.556 96.1136) (width 0.6096) (layer F.Cu) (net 3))
 (segment (start 128.1684 96.1136) (end 130.556 96.1136) (width 0.6096) (layer F.Cu) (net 3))
 (segment (start 130.556 96.1136) (end 133.4516 96.1136) (width 0.6096) (layer F.Cu) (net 3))
 (segment (start 133.4516 96.1136) (end 136.144 98.806) (width 0.6096) (layer F.Cu) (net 3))
 (segment (start 136.144 98.806) (end 136.144 100.076) (width 0.6096) (layer F.Cu) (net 3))
 (segment (start 136.144 100.076) (end 136.144 104.648) (width 0.6096) (layer F.Cu) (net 3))
 (segment (start 136.144 104.648) (end 136.398 104.902) (width 0.6096) (layer F.Cu) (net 3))
 (segment (start 125.984 96.1136) (end 128.1684 96.1136) (width 0.6096) (layer F.Cu) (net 3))
 (segment (start 152.4 105.283) (end 158.2166 105.283) (width 0.381) (layer F.Cu) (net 11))
 (segment (start 158.2166 105.283) (end 159.131 104.3686) (width 0.381) (layer F.Cu) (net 11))
 (segment (start 154.559 101.4095) (end 157.099 101.4095) (width 0.381) (layer F.Cu) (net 11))
 (segment (start 157.099 101.4095) (end 158.3055 101.4095) (width 0.381) (layer F.Cu) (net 11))
 (segment (start 158.3055 101.4095) (end 159.131 102.235) (width 0.381) (layer F.Cu) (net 11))
 (segment (start 131.064 85.852) (end 134.493 89.281) (width 0.381) (layer F.Cu) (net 11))
 (segment (start 159.131 98.171) (end 159.131 101.727) (width 0.381) (layer F.Cu) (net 11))
 (via blind (at 159.131 98.171) (size 1.016) (drill 0.508) (layers F.Cu B.Cu) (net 11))
 (segment (start 159.131 91.567) (end 159.131 98.171) (width 0.381) (layer B.Cu) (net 11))
 (segment (start 156.845 89.281) (end 159.131 91.567) (width 0.381) (layer B.Cu) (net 11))
 (segment (start 134.493 89.281) (end 156.845 89.281) (width 0.381) (layer B.Cu) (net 11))
 (via blind (at 134.493 89.281) (size 1.016) (drill 0.508) (layers F.Cu B.Cu) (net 11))
 (segment (start 146.304 111.252) (end 146.304 109.728) (width 0.381) (layer F.Cu) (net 11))
 (segment (start 159.131 104.3686) (end 159.131 102.235) (width 0.381) (layer F.Cu) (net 11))
 (segment (start 159.131 102.235) (end 159.131 101.727) (width 0.381) (layer F.Cu) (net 11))
 (segment (start 150.749 105.283) (end 152.4 105.283) (width 0.381) (layer F.Cu) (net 11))
 (segment (start 146.304 109.728) (end 150.749 105.283) (width 0.381) (layer F.Cu) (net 11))
 (segment (start 146.304 89.535) (end 146.304 90.17) (width 0.381) (layer F.Cu) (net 15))
 (segment (start 145.415 91.059) (end 145.415 92.075) (width 0.381) (layer F.Cu) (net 15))
 (segment (start 146.304 90.17) (end 145.415 91.059) (width 0.381) (layer F.Cu) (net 15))
 (segment (start 144.145 99.695) (end 144.145 93.345) (width 0.381) (layer B.Cu) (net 15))
 (segment (start 144.145 93.345) (end 145.415 92.075) (width 0.381) (layer B.Cu) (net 15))
 (via blind (at 145.415 92.075) (size 1.016) (drill 0.508) (layers F.Cu B.Cu) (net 15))
 (segment (start 141.224 111.252) (end 142.113 110.363) (width 0.381) (layer F.Cu) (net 15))
 (segment (start 142.113 101.727) (end 142.113 110.363) (width 0.381) (layer F.Cu) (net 15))
 (segment (start 144.145 99.695) (end 142.113 101.727) (width 0.381) (layer F.Cu) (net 15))
 (via blind (at 144.145 99.695) (size 1.016) (drill 0.508) (layers F.Cu B.Cu) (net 15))
 (segment (start 144.907 91.567) (end 143.57858 91.567) (width 0.381) (layer F.Cu) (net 15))
 (segment (start 145.415 92.075) (end 144.907 91.567) (width 0.381) (layer F.Cu) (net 15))
 (segment (start 146.304 85.852) (end 146.304 89.535) (width 0.381) (layer F.Cu) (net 15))
 (segment (start 146.304 89.535) (end 146.304 89.662) (width 0.381) (layer F.Cu) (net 15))
 (segment (start 154.559 99.5045) (end 154.559 98.425) (width 0.381) (layer F.Cu) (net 5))
 (segment (start 133.477 100.711) (end 131.953 100.711) (width 0.381) (layer F.Cu) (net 5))
 (segment (start 134.493 101.727) (end 133.477 100.711) (width 0.381) (layer F.Cu) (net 5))
 (via blind (at 134.493 101.727) (size 1.016) (drill 0.508) (layers F.Cu B.Cu) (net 5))
 (segment (start 148.209 101.727) (end 134.493 101.727) (width 0.381) (layer B.Cu) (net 5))
 (segment (start 152.019 97.917) (end 148.209 101.727) (width 0.381) (layer B.Cu) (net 5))
 (via blind (at 152.019 97.917) (size 1.016) (drill 0.508) (layers F.Cu B.Cu) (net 5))
 (segment (start 154.051 97.917) (end 152.019 97.917) (width 0.381) (layer F.Cu) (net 5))
 (segment (start 154.559 98.425) (end 154.051 97.917) (width 0.381) (layer F.Cu) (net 5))
 (segment (start 147.701 97.663) (end 148.209 98.171) (width 0.381) (layer F.Cu) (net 12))
 (segment (start 147.701 92.583) (end 147.701 91.059) (width 0.381) (layer B.Cu) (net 12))
 (via blind (at 147.701 97.663) (size 1.016) (drill 0.508) (layers F.Cu B.Cu) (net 12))
 (segment (start 147.701 97.663) (end 147.701 92.583) (width 0.381) (layer B.Cu) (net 12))
 (segment (start 148.463 90.297) (end 147.701 91.059) (width 0.381) (layer B.Cu) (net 12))
 (segment (start 150.6855 98.171) (end 152.019 99.5045) (width 0.381) (layer F.Cu) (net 12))
 (segment (start 148.209 98.171) (end 150.6855 98.171) (width 0.381) (layer F.Cu) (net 12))
 (segment (start 149.987 90.551) (end 156.591 90.551) (width 0.381) (layer F.Cu) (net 12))
 (via blind (at 149.987 90.551) (size 1.016) (drill 0.508) (layers F.Cu B.Cu) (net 12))
 (segment (start 157.099 91.059) (end 157.099 94.4245) (width 0.381) (layer F.Cu) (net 12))
 (segment (start 156.591 90.551) (end 157.099 91.059) (width 0.381) (layer F.Cu) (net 12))
 (segment (start 136.017 90.297) (end 148.463 90.297) (width 0.381) (layer B.Cu) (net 12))
 (segment (start 136.144 90.17) (end 136.017 90.297) (width 0.381) (layer F.Cu) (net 12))
 (via blind (at 136.017 90.297) (size 1.016) (drill 0.508) (layers F.Cu B.Cu) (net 12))
 (segment (start 136.144 85.852) (end 136.144 90.17) (width 0.381) (layer F.Cu) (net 12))
 (segment (start 148.463 90.297) (end 149.987 90.297) (width 0.381) (layer B.Cu) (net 12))
 (segment (start 136.144 85.852) (end 136.144 87.122) (width 0.381) (layer F.Cu) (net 12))
 (segment (start 157.099 92.329) (end 157.099 94.4245) (width 0.381) (layer F.Cu) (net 12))
 (segment (start 147.193 102.6414) (end 147.193 103.8606) (width 0.381) (layer F.Cu) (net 2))
 (segment (start 147.8534 104.521) (end 148.717 104.521) (width 0.381) (layer F.Cu) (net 2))
 (segment (start 147.193 103.8606) (end 147.8534 104.521) (width 0.381) (layer F.Cu) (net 2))
 (segment (start 147.193 100.711) (end 147.193 102.6414) (width 0.381) (layer F.Cu) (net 2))
 (segment (start 148.717 104.521) (end 151.511 104.521) (width 0.381) (layer F.Cu) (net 2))
 (segment (start 151.511 104.521) (end 152.019 104.013) (width 0.381) (layer F.Cu) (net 2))
 (segment (start 152.019 104.013) (end 152.019 101.4095) (width 0.381) (layer F.Cu) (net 2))
 (segment (start 131.953 93.091) (end 133.985 93.091) (width 0.381) (layer F.Cu) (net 2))
 (via blind (at 147.193 100.711) (size 1.016) (drill 0.508) (layers F.Cu B.Cu) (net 2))
 (segment (start 143.383 100.711) (end 147.193 100.711) (width 0.381) (layer B.Cu) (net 2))
 (segment (start 142.621 99.949) (end 143.383 100.711) (width 0.381) (layer B.Cu) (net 2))
 (segment (start 142.621 96.901) (end 142.621 99.949) (width 0.381) (layer B.Cu) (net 2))
 (segment (start 140.081 94.361) (end 142.621 96.901) (width 0.381) (layer B.Cu) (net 2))
 (segment (start 135.255 94.361) (end 140.081 94.361) (width 0.381) (layer B.Cu) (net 2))
 (segment (start 134.747 93.853) (end 135.255 94.361) (width 0.381) (layer B.Cu) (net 2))
 (via blind (at 134.747 93.853) (size 1.016) (drill 0.508) (layers F.Cu B.Cu) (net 2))
 (segment (start 133.985 93.091) (end 134.747 93.853) (width 0.381) (layer F.Cu) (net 2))
 (segment (start 120.904 95.25) (end 120.904 98.679) (width 0.6096) (layer F.Cu) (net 4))
 (segment (start 121.9454 99.7204) (end 125.984 99.7204) (width 0.6096) (layer F.Cu) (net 4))
 (segment (start 120.904 98.679) (end 121.9454 99.7204) (width 0.6096) (layer F.Cu) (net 4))
 (segment (start 125.984 99.7204) (end 129.1844 99.7204) (width 0.6096) (layer F.Cu) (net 4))
 (segment (start 129.1844 99.7204) (end 130.175 100.711) (width 0.6096) (layer F.Cu) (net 4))
 (segment (start 120.904 85.852) (end 120.904 95.25) (width 0.6096) (layer F.Cu) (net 4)))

